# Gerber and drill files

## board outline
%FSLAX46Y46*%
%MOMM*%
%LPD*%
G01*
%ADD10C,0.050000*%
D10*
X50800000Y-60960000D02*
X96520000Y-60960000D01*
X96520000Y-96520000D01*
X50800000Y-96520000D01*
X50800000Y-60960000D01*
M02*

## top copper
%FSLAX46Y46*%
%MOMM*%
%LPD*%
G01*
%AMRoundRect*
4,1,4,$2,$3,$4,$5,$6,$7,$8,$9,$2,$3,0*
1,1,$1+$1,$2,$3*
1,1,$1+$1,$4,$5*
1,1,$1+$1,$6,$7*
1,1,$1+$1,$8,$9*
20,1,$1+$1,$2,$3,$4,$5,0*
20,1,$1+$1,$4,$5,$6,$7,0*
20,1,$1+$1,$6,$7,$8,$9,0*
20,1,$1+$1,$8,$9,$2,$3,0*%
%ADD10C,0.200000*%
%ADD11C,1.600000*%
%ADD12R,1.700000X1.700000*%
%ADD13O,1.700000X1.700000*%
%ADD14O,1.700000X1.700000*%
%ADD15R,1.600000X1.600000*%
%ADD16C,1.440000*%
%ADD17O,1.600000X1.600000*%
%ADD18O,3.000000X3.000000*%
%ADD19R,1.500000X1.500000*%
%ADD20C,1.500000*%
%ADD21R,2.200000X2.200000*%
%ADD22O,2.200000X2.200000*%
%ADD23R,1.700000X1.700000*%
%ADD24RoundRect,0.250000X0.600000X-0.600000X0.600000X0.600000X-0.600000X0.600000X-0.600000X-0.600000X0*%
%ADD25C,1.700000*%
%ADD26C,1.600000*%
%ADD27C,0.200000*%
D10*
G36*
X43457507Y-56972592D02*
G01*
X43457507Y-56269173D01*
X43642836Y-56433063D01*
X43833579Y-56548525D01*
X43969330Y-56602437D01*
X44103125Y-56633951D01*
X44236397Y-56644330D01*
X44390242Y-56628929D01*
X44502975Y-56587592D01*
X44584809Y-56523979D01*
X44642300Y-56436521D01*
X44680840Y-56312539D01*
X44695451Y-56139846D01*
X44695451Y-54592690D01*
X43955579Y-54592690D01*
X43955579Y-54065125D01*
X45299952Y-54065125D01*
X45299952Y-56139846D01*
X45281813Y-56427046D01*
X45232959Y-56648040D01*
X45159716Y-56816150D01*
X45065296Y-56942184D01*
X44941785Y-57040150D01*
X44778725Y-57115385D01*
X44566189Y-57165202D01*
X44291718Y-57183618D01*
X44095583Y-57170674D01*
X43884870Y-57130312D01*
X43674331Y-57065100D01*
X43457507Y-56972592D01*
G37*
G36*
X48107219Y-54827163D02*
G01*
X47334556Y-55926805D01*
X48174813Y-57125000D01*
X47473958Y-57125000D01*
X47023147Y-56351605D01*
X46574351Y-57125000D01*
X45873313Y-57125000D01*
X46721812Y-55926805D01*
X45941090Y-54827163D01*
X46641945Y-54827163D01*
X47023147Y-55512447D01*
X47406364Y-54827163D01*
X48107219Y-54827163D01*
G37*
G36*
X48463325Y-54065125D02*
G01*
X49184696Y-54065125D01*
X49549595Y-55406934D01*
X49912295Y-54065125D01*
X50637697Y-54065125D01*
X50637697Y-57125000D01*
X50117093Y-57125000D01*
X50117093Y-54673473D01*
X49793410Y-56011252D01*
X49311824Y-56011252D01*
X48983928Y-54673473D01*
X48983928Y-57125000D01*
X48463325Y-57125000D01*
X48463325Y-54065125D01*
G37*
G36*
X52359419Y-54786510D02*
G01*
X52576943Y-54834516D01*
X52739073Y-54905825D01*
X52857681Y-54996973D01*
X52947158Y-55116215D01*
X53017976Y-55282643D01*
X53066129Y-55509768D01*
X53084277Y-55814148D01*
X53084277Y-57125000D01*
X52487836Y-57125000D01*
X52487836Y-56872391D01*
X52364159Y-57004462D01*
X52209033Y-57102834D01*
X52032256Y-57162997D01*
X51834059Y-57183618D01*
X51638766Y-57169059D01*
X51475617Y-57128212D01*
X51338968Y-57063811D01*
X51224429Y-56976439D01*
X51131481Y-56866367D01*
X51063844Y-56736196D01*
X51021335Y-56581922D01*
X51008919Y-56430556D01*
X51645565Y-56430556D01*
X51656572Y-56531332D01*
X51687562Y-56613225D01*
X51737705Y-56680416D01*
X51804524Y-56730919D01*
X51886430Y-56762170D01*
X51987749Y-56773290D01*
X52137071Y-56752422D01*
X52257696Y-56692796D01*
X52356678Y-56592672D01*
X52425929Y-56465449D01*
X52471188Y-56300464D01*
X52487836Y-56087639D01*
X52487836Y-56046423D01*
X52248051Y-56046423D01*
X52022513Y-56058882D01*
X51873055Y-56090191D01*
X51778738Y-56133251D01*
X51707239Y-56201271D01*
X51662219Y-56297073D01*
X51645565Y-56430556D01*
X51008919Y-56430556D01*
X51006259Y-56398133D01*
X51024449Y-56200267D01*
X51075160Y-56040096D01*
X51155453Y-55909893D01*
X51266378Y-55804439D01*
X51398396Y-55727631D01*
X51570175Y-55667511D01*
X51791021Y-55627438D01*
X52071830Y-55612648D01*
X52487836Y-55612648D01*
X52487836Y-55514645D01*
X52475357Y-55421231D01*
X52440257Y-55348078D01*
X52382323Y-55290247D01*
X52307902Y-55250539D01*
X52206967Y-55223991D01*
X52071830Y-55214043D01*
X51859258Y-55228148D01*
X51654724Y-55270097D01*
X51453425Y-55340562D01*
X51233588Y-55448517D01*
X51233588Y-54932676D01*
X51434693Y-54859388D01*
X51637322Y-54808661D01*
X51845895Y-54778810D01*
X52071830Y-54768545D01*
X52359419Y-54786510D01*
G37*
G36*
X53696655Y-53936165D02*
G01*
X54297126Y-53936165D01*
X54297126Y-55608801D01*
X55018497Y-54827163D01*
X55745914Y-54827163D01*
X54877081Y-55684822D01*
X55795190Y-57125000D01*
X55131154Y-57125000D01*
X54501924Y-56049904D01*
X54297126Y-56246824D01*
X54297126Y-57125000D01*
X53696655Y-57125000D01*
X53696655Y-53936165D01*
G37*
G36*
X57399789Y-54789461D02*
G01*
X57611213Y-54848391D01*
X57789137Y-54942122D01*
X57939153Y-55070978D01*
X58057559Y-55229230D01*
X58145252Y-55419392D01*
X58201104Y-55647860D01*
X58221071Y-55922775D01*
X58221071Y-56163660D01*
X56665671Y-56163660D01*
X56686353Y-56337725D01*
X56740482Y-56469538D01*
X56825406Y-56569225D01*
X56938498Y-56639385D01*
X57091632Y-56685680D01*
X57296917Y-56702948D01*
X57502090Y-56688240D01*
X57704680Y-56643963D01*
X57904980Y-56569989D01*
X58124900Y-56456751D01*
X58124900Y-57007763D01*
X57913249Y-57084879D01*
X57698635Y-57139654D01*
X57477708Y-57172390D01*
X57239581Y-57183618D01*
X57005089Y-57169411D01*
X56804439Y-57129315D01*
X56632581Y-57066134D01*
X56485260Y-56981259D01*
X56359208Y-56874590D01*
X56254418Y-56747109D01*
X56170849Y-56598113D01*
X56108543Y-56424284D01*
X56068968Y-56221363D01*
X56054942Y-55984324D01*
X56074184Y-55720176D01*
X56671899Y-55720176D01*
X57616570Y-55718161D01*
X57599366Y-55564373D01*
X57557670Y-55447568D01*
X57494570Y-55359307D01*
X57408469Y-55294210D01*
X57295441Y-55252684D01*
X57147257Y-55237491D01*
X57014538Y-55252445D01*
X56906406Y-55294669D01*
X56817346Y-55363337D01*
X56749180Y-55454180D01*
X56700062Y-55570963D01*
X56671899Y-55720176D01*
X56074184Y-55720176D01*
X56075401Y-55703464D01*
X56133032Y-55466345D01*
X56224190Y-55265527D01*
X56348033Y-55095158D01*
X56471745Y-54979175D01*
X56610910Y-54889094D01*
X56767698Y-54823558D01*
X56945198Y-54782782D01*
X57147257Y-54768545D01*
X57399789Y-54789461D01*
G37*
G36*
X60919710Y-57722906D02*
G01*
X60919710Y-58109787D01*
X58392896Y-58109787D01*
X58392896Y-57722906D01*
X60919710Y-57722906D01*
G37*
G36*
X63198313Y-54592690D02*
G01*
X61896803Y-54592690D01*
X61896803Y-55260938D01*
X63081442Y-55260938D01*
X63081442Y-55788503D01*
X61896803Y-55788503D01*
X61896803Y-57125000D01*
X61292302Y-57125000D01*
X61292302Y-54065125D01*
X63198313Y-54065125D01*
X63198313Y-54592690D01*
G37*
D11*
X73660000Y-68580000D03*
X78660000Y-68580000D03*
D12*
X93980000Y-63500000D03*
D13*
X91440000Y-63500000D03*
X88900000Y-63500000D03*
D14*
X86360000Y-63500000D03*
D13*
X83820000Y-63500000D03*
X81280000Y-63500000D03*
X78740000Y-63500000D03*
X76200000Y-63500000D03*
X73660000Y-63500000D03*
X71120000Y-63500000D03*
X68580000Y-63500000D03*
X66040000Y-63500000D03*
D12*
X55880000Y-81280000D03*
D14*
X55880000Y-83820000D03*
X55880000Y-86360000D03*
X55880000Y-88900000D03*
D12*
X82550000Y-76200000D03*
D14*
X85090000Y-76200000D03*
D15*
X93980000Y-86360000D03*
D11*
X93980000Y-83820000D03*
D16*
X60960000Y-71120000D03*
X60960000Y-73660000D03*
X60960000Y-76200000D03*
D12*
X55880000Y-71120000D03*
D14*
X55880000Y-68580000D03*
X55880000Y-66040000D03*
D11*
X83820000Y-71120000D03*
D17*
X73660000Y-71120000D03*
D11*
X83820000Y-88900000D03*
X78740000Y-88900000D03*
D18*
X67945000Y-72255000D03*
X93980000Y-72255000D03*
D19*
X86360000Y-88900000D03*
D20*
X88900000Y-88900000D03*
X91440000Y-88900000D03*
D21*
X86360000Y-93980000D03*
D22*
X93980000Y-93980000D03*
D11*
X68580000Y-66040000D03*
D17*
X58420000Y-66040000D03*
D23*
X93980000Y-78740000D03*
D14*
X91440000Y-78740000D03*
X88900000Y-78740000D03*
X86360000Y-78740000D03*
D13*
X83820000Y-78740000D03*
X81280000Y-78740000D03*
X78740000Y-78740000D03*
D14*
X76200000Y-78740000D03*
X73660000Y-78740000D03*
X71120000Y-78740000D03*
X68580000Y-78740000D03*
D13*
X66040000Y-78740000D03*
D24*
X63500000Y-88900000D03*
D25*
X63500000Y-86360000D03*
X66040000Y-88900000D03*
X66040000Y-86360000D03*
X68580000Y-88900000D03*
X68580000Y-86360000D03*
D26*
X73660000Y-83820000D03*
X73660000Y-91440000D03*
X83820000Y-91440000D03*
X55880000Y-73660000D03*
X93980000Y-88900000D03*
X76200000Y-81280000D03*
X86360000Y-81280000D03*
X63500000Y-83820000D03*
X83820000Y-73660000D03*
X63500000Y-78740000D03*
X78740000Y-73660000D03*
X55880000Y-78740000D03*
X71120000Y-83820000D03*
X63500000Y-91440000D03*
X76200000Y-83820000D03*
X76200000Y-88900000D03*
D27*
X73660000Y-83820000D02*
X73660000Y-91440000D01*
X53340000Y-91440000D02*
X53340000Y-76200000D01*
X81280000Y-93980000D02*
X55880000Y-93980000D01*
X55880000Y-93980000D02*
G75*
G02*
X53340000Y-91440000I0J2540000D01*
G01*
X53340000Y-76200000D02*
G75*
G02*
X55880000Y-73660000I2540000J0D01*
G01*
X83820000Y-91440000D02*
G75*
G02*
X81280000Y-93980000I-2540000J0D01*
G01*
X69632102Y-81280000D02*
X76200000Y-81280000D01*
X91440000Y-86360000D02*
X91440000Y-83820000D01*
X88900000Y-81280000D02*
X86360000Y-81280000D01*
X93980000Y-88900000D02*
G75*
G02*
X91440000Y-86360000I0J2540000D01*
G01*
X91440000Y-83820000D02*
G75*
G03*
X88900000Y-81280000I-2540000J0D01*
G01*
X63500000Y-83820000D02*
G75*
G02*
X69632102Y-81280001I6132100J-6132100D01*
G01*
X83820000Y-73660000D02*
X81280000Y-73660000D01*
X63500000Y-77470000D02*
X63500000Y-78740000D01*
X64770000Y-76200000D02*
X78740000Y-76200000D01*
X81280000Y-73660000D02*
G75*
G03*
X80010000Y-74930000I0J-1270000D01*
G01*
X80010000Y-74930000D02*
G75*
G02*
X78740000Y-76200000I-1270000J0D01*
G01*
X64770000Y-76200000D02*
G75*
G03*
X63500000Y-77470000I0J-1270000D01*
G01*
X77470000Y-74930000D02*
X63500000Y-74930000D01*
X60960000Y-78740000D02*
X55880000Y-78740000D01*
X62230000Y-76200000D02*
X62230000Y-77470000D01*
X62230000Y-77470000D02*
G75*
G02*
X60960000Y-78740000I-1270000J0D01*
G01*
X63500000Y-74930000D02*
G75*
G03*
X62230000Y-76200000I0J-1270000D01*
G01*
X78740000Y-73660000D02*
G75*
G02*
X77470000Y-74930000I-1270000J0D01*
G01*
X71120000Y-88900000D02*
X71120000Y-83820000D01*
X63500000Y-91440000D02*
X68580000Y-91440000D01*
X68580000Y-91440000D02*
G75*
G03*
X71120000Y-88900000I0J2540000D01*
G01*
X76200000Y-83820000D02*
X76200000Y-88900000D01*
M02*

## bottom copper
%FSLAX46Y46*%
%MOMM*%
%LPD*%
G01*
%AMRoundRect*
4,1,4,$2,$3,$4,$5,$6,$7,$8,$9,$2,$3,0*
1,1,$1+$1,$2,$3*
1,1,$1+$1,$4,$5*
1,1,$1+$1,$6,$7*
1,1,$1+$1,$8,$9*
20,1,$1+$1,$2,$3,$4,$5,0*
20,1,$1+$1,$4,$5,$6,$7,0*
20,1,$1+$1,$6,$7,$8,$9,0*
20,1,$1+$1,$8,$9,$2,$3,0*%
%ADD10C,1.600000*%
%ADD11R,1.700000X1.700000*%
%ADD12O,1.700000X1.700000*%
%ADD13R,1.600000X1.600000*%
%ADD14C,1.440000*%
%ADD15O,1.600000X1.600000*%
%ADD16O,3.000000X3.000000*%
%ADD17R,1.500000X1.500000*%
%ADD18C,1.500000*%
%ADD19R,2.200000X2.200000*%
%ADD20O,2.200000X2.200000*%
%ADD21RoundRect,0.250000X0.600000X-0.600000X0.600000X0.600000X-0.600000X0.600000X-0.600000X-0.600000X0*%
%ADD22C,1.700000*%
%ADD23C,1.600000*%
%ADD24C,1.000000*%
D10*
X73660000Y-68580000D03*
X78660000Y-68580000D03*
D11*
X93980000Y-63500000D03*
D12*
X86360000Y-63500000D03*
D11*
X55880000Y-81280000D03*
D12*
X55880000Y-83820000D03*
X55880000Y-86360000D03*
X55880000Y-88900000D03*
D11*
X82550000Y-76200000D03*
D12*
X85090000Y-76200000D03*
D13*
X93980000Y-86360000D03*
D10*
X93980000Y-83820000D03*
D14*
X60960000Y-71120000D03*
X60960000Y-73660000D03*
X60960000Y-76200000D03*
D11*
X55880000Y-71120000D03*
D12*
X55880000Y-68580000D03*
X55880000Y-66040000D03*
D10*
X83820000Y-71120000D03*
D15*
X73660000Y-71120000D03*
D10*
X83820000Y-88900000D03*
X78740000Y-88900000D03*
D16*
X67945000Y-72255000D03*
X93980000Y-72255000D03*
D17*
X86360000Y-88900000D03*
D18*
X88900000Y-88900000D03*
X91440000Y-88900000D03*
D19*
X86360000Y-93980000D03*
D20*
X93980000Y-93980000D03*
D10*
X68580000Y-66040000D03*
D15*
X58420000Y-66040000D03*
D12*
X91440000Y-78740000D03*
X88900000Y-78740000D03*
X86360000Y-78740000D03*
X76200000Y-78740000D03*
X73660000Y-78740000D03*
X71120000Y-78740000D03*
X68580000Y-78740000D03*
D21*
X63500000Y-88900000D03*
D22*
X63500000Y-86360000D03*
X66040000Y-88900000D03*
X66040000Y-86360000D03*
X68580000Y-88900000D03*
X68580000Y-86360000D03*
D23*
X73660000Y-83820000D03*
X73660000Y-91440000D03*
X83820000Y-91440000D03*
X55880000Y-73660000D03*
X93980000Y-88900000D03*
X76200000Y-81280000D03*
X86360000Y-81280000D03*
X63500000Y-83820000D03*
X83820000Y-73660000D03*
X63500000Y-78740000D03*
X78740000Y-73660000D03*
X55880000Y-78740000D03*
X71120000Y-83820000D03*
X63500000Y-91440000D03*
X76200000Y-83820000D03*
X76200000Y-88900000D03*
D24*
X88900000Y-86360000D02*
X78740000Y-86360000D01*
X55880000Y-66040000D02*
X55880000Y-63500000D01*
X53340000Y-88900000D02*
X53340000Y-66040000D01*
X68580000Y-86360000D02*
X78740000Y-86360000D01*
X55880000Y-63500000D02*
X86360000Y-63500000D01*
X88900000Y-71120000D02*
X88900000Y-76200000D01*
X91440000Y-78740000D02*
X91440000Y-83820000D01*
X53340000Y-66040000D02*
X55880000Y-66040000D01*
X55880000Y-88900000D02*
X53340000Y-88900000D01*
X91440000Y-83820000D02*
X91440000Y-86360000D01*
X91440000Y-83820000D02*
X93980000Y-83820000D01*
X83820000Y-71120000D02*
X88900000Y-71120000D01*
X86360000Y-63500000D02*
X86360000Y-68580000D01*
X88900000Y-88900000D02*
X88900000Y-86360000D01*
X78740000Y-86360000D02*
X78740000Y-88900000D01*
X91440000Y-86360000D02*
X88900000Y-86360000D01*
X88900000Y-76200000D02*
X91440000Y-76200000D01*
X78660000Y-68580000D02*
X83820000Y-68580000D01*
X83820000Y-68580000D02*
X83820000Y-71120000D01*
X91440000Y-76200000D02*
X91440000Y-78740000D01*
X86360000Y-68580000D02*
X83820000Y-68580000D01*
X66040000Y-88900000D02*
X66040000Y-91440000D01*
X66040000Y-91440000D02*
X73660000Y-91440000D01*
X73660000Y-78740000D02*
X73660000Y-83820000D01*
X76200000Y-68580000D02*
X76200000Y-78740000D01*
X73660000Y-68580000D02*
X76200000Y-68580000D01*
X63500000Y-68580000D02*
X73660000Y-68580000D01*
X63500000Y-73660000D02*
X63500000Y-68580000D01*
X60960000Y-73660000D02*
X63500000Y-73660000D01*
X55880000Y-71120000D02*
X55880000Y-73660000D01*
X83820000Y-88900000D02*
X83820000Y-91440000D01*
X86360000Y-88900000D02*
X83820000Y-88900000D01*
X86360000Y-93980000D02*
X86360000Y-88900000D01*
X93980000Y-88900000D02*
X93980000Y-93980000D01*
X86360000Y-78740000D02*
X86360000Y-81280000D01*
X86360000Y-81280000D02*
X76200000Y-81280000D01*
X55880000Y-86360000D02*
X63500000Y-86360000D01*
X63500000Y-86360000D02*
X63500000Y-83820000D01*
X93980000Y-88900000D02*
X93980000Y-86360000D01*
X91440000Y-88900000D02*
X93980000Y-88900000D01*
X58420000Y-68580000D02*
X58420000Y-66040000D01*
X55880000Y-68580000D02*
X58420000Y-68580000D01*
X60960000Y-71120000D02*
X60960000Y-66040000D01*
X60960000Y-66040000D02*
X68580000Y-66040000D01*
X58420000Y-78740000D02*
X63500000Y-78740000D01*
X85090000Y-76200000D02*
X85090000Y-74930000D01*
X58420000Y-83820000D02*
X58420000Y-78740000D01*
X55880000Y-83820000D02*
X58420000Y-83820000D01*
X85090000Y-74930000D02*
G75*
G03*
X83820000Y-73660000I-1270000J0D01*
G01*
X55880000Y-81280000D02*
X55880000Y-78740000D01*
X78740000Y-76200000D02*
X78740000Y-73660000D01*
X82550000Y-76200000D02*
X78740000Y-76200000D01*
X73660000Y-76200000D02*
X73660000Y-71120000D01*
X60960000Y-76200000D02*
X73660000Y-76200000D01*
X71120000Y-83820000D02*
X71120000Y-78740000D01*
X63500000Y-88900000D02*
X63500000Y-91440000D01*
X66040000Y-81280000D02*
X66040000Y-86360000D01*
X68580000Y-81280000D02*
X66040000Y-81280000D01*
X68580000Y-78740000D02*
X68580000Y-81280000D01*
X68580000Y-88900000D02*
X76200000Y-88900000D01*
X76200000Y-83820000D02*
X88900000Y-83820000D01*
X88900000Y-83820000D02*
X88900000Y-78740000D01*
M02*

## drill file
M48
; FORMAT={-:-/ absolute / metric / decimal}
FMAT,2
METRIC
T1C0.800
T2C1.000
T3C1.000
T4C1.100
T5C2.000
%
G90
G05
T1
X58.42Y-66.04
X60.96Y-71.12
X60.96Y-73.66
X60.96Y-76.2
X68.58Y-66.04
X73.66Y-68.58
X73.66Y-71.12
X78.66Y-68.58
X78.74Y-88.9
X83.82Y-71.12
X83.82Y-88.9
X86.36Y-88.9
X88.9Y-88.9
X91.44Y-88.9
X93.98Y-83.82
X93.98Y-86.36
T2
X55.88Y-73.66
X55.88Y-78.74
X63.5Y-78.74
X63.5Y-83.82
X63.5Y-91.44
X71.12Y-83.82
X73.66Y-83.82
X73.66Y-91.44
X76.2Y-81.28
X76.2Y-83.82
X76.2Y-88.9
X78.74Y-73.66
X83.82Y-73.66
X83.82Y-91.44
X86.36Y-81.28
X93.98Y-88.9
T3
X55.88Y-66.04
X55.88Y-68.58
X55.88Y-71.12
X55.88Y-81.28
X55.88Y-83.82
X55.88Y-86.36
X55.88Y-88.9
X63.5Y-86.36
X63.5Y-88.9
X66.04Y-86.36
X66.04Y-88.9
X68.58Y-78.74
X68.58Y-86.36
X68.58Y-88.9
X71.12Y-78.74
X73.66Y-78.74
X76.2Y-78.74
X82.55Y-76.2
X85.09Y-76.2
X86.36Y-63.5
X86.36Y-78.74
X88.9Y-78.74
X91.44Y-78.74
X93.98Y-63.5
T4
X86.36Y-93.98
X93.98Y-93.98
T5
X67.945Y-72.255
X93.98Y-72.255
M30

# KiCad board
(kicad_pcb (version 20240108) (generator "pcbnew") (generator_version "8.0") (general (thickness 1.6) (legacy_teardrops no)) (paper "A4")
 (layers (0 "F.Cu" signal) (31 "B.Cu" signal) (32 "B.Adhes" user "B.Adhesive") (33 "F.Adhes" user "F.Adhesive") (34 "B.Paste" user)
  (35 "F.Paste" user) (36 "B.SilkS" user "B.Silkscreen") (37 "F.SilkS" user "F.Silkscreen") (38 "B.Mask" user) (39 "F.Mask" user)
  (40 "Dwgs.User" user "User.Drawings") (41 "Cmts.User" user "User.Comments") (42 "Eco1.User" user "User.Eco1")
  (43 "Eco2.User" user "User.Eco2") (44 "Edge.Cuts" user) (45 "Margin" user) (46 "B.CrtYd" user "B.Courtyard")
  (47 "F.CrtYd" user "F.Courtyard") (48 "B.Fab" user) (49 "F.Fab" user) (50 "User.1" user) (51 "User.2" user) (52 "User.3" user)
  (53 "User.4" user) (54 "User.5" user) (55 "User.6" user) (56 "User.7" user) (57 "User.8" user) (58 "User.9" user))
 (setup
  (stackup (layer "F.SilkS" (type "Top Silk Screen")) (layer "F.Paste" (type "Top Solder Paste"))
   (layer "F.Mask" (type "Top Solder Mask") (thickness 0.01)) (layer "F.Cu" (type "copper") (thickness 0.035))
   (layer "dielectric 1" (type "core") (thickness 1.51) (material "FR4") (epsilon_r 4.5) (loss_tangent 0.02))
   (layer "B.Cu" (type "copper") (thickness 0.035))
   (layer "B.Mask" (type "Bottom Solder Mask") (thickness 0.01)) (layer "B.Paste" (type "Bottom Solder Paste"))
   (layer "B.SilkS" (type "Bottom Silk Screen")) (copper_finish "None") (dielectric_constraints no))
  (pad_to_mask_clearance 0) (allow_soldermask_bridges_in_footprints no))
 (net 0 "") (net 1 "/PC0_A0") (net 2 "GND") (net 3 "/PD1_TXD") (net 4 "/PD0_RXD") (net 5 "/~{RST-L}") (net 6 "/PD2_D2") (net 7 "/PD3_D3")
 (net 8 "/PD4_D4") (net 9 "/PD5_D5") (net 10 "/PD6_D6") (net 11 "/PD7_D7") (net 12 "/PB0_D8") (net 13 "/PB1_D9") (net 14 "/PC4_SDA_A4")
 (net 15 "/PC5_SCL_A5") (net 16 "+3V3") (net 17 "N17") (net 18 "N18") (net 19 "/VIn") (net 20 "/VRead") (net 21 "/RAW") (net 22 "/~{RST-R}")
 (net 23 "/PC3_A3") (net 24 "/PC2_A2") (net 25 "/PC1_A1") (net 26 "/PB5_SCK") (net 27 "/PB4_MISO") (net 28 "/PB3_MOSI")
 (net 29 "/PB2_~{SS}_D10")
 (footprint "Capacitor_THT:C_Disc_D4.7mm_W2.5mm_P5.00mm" (layer "F.Cu") (at 73.66 68.58)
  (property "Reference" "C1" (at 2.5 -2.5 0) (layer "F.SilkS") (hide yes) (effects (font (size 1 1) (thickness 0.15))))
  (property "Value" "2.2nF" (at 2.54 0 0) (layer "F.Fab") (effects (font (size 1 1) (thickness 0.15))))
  (pad "1" thru_hole circle (at 0 0) (size 1.6 1.6) (drill 0.8) (layers "*.Cu" "*.Mask") (remove_unused_layers yes) (keep_end_layers yes)
   (zone_layer_connections) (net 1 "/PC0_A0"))
  (pad "2" thru_hole circle (at 5 0) (size 1.6 1.6) (drill 0.8) (layers "*.Cu" "*.Mask") (remove_unused_layers yes) (keep_end_layers yes)
   (zone_layer_connections) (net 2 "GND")))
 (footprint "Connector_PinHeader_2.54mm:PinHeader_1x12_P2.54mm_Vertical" (layer "F.Cu") (at 93.98 63.5 -90)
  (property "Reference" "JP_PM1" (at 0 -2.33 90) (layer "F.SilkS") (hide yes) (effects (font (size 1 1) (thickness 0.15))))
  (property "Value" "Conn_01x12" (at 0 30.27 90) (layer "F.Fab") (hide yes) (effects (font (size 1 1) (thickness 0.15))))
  (pad "1" thru_hole rect (at 0 0 270) (size 1.7 1.7) (drill 1) (layers "*.Cu" "*.Mask") (remove_unused_layers yes) (keep_end_layers yes)
   (zone_layer_connections) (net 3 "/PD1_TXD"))
  (pad "2" smd oval (at 0 2.54 270) (size 1.7 1.7) (layers "F.Cu" "F.Paste" "F.Mask") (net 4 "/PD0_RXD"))
  (pad "3" smd oval (at 0 5.08 270) (size 1.7 1.7) (layers "F.Cu" "F.Paste" "F.Mask") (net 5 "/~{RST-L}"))
  (pad "4" thru_hole oval (at 0 7.62 270) (size 1.7 1.7) (drill 1) (layers "*.Cu" "*.Mask") (remove_unused_layers yes) (keep_end_layers yes)
   (zone_layer_connections) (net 2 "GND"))
  (pad "5" smd oval (at 0 10.16 270) (size 1.7 1.7) (layers "F.Cu" "F.Paste" "F.Mask") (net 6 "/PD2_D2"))
  (pad "6" smd oval (at 0 12.7 270) (size 1.7 1.7) (layers "F.Cu" "F.Paste" "F.Mask") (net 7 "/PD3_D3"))
  (pad "7" smd oval (at 0 15.24 270) (size 1.7 1.7) (layers "F.Cu" "F.Paste" "F.Mask") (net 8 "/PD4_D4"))
  (pad "8" smd oval (at 0 17.78 270) (size 1.7 1.7) (layers "F.Cu" "F.Paste" "F.Mask") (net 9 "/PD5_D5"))
  (pad "9" smd oval (at 0 20.32 270) (size 1.7 1.7) (layers "F.Cu" "F.Paste" "F.Mask") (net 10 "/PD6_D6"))
  (pad "10" smd oval (at 0 22.86 270) (size 1.7 1.7) (layers "F.Cu" "F.Paste" "F.Mask") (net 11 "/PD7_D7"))
  (pad "11" smd oval (at 0 25.4 270) (size 1.7 1.7) (layers "F.Cu" "F.Paste" "F.Mask") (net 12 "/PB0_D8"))
  (pad "12" smd oval (at 0 27.94 270) (size 1.7 1.7) (layers "F.Cu" "F.Paste" "F.Mask") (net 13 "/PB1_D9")))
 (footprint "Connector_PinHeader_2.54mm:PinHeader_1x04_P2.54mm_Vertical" (layer "F.Cu") (at 55.88 81.28)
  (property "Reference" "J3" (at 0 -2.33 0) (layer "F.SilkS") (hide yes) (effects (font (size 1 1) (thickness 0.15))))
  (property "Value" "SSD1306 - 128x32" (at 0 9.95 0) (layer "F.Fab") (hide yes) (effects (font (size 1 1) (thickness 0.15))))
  (pad "1" thru_hole rect (at 0 0) (size 1.7 1.7) (drill 1) (layers "*.Cu" "*.Mask") (remove_unused_layers yes) (keep_end_layers yes)
   (zone_layer_connections) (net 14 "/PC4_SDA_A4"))
  (pad "2" thru_hole oval (at 0 2.54) (size 1.7 1.7) (drill 1) (layers "*.Cu" "*.Mask") (remove_unused_layers yes) (keep_end_layers yes)
   (zone_layer_connections) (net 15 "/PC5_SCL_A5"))
  (pad "3" thru_hole oval (at 0 5.08) (size 1.7 1.7) (drill 1) (layers "*.Cu" "*.Mask") (remove_unused_layers yes) (keep_end_layers yes)
   (zone_layer_connections) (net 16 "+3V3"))
  (pad "4" thru_hole oval (at 0 7.62) (size 1.7 1.7) (drill 1) (layers "*.Cu" "*.Mask") (remove_unused_layers yes) (keep_end_layers yes)
   (zone_layer_connections) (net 2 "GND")))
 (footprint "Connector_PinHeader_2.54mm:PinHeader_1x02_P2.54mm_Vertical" (layer "F.Cu") (at 82.55 76.2 90)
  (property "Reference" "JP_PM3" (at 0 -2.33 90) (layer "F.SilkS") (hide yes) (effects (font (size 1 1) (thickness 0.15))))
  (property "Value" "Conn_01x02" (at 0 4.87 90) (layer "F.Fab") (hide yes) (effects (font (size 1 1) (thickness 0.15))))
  (pad "1" thru_hole rect (at 0 0 90) (size 1.7 1.7) (drill 1) (layers "*.Cu" "*.Mask") (remove_unused_layers yes) (keep_end_layers yes)
   (zone_layer_connections) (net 14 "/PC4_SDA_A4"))
  (pad "2" thru_hole oval (at 0 2.54 90) (size 1.7 1.7) (drill 1) (layers "*.Cu" "*.Mask") (remove_unused_layers yes) (keep_end_layers yes)
   (zone_layer_connections) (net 15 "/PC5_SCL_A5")))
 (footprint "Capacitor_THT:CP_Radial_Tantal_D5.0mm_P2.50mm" (layer "F.Cu") (at 93.98 86.36 90)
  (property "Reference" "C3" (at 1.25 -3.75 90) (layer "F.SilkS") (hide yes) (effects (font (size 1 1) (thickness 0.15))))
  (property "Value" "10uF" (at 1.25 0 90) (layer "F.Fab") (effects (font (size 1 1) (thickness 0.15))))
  (pad "1" thru_hole rect (at 0 0 90) (size 1.6 1.6) (drill 0.8) (layers "*.Cu" "*.Mask") (remove_unused_layers yes) (keep_end_layers yes)
   (zone_layer_connections) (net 16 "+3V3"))
  (pad "2" thru_hole circle (at 2.54 0 90) (size 1.6 1.6) (drill 0.8) (layers "*.Cu" "*.Mask") (remove_unused_layers yes)
   (keep_end_layers yes) (zone_layer_connections) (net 2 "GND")))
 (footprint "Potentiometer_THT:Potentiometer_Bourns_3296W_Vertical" (layer "F.Cu") (at 60.96 71.12 90)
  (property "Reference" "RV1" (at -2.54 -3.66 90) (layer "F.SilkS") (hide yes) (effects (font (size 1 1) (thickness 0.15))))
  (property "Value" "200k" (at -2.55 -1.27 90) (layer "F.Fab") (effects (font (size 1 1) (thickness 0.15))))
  (pad "1" thru_hole circle (at 0 0 90) (size 1.44 1.44) (drill 0.8) (layers "*.Cu" "*.Mask") (remove_unused_layers yes)
   (keep_end_layers yes) (zone_layer_connections) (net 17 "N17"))
  (pad "2" thru_hole circle (at -2.54 0 90) (size 1.44 1.44) (drill 0.8) (layers "*.Cu" "*.Mask") (remove_unused_layers yes)
   (keep_end_layers yes) (zone_layer_connections) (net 1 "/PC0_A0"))
  (pad "3" thru_hole circle (at -5.08 0 90) (size 1.44 1.44) (drill 0.8) (layers "*.Cu" "*.Mask") (remove_unused_layers yes)
   (keep_end_layers yes) (zone_layer_connections) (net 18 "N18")))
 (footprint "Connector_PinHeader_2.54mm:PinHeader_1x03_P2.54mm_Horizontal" (layer "F.Cu") (at 55.88 71.12 180)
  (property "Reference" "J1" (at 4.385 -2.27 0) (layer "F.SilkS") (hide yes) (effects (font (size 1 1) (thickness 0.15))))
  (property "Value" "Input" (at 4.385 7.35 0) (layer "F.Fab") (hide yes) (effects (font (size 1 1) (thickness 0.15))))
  (pad "1" thru_hole rect (at 0 0 180) (size 1.7 1.7) (drill 1) (layers "*.Cu" "*.Mask") (remove_unused_layers yes) (keep_end_layers yes)
   (zone_layer_connections) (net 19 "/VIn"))
  (pad "2" thru_hole oval (at 0 2.54 180) (size 1.7 1.7) (drill 1) (layers "*.Cu" "*.Mask") (remove_unused_layers yes) (keep_end_layers yes)
   (zone_layer_connections) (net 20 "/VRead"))
  (pad "3" thru_hole oval (at 0 5.08 180) (size 1.7 1.7) (drill 1) (layers "*.Cu" "*.Mask") (remove_unused_layers yes) (keep_end_layers yes)
   (zone_layer_connections) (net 2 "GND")))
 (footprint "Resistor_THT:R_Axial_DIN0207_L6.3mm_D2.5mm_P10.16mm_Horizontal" (layer "F.Cu") (at 83.82 71.12 180)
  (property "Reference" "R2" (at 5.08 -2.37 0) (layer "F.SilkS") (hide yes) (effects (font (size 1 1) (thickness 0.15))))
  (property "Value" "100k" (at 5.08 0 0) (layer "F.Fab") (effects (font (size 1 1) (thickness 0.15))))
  (pad "1" thru_hole circle (at 0 0 180) (size 1.6 1.6) (drill 0.8) (layers "*.Cu" "*.Mask") (remove_unused_layers yes)
   (keep_end_layers yes) (zone_layer_connections) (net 2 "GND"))
  (pad "2" thru_hole oval (at 10.16 0 180) (size 1.6 1.6) (drill 0.8) (layers "*.Cu" "*.Mask") (remove_unused_layers yes)
   (keep_end_layers yes) (zone_layer_connections) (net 18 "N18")))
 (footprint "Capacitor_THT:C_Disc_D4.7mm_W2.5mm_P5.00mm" (layer "F.Cu") (at 83.82 88.9 180)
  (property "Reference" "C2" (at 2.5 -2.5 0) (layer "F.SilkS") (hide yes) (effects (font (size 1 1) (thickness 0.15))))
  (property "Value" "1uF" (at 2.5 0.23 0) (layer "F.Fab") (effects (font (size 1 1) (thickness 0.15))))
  (pad "1" thru_hole circle (at 0 0 180) (size 1.6 1.6) (drill 0.8) (layers "*.Cu" "*.Mask") (remove_unused_layers yes)
   (keep_end_layers yes) (zone_layer_connections) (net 19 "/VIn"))
  (pad "2" thru_hole circle (at 5.08 0 180) (size 1.6 1.6) (drill 0.8) (layers "*.Cu" "*.Mask") (remove_unused_layers yes)
   (keep_end_layers yes) (zone_layer_connections) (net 2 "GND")))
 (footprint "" (layer "F.Cu") (at 67.945 72.255)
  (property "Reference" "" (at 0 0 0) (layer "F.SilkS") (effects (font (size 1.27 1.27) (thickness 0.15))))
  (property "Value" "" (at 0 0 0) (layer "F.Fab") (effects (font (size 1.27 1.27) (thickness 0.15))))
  (pad "1" thru_hole oval (at 0 0 90) (size 3 3) (drill 2) (layers "*.Cu" "*.Mask") (remove_unused_layers yes) (keep_end_layers yes)
   (zone_layer_connections))
  (pad "2" thru_hole oval (at 26.035 0 90) (size 3 3) (drill 2) (layers "*.Cu" "*.Mask") (remove_unused_layers yes) (keep_end_layers yes)
   (zone_layer_connections)))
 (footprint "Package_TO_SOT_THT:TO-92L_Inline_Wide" (layer "F.Cu") (at 86.36 88.9)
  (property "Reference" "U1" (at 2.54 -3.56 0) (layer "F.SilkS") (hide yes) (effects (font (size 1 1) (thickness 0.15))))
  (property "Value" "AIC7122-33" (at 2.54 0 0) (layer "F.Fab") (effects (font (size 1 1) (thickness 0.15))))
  (pad "1" thru_hole rect (at 0 0) (size 1.5 1.5) (drill 0.8) (layers "*.Cu" "*.Mask") (remove_unused_layers yes) (keep_end_layers yes)
   (zone_layer_connections) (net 19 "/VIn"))
  (pad "2" thru_hole circle (at 2.54 0) (size 1.5 1.5) (drill 0.8) (layers "*.Cu" "*.Mask") (remove_unused_layers yes) (keep_end_layers yes)
   (zone_layer_connections) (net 2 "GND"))
  (pad "3" thru_hole circle (at 5.08 0) (size 1.5 1.5) (drill 0.8) (layers "*.Cu" "*.Mask") (remove_unused_layers yes) (keep_end_layers yes)
   (zone_layer_connections) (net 16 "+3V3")))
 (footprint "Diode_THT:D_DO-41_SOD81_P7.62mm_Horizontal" (layer "F.Cu") (at 86.36 93.98)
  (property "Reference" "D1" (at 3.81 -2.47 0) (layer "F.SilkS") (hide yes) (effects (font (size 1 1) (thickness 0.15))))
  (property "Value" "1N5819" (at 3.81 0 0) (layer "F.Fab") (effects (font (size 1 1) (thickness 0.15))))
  (pad "1" thru_hole rect (at 0 0) (size 2.2 2.2) (drill 1.1) (layers "*.Cu" "*.Mask") (remove_unused_layers no) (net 19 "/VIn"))
  (pad "2" thru_hole oval (at 7.62 0) (size 2.2 2.2) (drill 1.1) (layers "*.Cu" "*.Mask") (remove_unused_layers no) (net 16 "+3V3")))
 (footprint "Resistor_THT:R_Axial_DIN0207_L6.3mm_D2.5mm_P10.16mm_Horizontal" (layer "F.Cu") (at 68.58 66.04 180)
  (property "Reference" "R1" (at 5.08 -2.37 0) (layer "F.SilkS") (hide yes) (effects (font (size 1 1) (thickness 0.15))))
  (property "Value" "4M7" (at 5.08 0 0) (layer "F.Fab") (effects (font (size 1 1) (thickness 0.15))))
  (pad "1" thru_hole circle (at 0 0 180) (size 1.6 1.6) (drill 0.8) (layers "*.Cu" "*.Mask") (remove_unused_layers yes)
   (keep_end_layers yes) (zone_layer_connections) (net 17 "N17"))
  (pad "2" thru_hole oval (at 10.16 0 180) (size 1.6 1.6) (drill 0.8) (layers "*.Cu" "*.Mask") (remove_unused_layers yes)
   (keep_end_layers yes) (zone_layer_connections) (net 20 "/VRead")))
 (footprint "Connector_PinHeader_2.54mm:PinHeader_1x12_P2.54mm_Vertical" (layer "F.Cu") (at 93.98 78.74 -90)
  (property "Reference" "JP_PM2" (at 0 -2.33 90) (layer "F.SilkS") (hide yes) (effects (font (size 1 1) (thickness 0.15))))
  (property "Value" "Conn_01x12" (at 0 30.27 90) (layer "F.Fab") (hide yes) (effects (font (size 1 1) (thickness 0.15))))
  (pad "1" smd rect (at 0 0 270) (size 1.7 1.7) (layers "F.Cu" "F.Paste" "F.Mask") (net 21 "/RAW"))
  (pad "2" thru_hole oval (at 0 2.54 270) (size 1.7 1.7) (drill 1) (layers "*.Cu" "*.Mask") (remove_unused_layers yes) (keep_end_layers yes)
   (zone_layer_connections) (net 2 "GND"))
  (pad "3" thru_hole oval (at 0 5.08 270) (size 1.7 1.7) (drill 1) (layers "*.Cu" "*.Mask") (remove_unused_layers yes) (keep_end_layers yes)
   (zone_layer_connections) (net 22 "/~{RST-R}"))
  (pad "4" thru_hole oval (at 0 7.62 270) (size 1.7 1.7) (drill 1) (layers "*.Cu" "*.Mask") (remove_unused_layers yes) (keep_end_layers yes)
   (zone_layer_connections) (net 16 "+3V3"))
  (pad "5" smd oval (at 0 10.16 270) (size 1.7 1.7) (layers "F.Cu" "F.Paste" "F.Mask") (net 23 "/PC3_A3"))
  (pad "6" smd oval (at 0 12.7 270) (size 1.7 1.7) (layers "F.Cu" "F.Paste" "F.Mask") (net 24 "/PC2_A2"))
  (pad "7" smd oval (at 0 15.24 270) (size 1.7 1.7) (layers "F.Cu" "F.Paste" "F.Mask") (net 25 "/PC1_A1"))
  (pad "8" thru_hole oval (at 0 17.78 270) (size 1.7 1.7) (drill 1) (layers "*.Cu" "*.Mask") (remove_unused_layers yes)
   (keep_end_layers yes) (zone_layer_connections) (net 1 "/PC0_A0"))
  (pad "9" thru_hole oval (at 0 20.32 270) (size 1.7 1.7) (drill 1) (layers "*.Cu" "*.Mask") (remove_unused_layers yes)
   (keep_end_layers yes) (zone_layer_connections) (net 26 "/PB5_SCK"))
  (pad "10" thru_hole oval (at 0 22.86 270) (size 1.7 1.7) (drill 1) (layers "*.Cu" "*.Mask") (remove_unused_layers yes)
   (keep_end_layers yes) (zone_layer_connections) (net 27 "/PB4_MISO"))
  (pad "11" thru_hole oval (at 0 25.4 270) (size 1.7 1.7) (drill 1) (layers "*.Cu" "*.Mask") (remove_unused_layers yes)
   (keep_end_layers yes) (zone_layer_connections) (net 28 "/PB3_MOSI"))
  (pad "12" smd oval (at 0 27.94 270) (size 1.7 1.7) (layers "F.Cu" "F.Paste" "F.Mask") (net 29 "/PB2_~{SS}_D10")))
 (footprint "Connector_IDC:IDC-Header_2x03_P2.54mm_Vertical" (layer "F.Cu") (at 63.5 88.9 90)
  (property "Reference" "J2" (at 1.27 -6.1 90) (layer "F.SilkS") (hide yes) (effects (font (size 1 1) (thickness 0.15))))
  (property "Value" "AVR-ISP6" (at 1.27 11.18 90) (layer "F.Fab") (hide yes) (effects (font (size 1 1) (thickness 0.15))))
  (pad "1" thru_hole roundrect (at 0 0 90) (size 1.7 1.7) (drill 1) (layers "*.Cu" "*.Mask") (remove_unused_layers yes)
   (keep_end_layers yes) (zone_layer_connections) (roundrect_rratio 0.147059) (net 27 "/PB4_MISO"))
  (pad "2" thru_hole circle (at 2.54 0 90) (size 1.7 1.7) (drill 1) (layers "*.Cu" "*.Mask") (remove_unused_layers yes)
   (keep_end_layers yes) (zone_layer_connections) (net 16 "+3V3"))
  (pad "3" thru_hole circle (at 0 2.54 90) (size 1.7 1.7) (drill 1) (layers "*.Cu" "*.Mask") (remove_unused_layers yes)
   (keep_end_layers yes) (zone_layer_connections) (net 26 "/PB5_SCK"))
  (pad "4" thru_hole circle (at 2.54 2.54 90) (size 1.7 1.7) (drill 1) (layers "*.Cu" "*.Mask") (remove_unused_layers yes)
   (keep_end_layers yes) (zone_layer_connections) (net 28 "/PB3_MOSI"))
  (pad "5" thru_hole circle (at 0 5.08 90) (size 1.7 1.7) (drill 1) (layers "*.Cu" "*.Mask") (remove_unused_layers yes)
   (keep_end_layers yes) (zone_layer_connections) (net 22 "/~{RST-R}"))
  (pad "6" thru_hole circle (at 2.54 5.08 90) (size 1.7 1.7) (drill 1) (layers "*.Cu" "*.Mask") (remove_unused_layers yes)
   (keep_end_layers yes) (zone_layer_connections) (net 2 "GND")))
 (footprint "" (layer "F.Cu") (at 106.553 77.851)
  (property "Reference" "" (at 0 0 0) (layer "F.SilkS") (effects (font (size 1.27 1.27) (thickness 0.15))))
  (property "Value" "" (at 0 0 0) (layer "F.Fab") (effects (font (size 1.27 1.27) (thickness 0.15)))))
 (gr_rect (start 50.8 60.96) (end 96.52 96.52) (stroke (width 0.05) (type default)) (fill none) (layer "Edge.Cuts"))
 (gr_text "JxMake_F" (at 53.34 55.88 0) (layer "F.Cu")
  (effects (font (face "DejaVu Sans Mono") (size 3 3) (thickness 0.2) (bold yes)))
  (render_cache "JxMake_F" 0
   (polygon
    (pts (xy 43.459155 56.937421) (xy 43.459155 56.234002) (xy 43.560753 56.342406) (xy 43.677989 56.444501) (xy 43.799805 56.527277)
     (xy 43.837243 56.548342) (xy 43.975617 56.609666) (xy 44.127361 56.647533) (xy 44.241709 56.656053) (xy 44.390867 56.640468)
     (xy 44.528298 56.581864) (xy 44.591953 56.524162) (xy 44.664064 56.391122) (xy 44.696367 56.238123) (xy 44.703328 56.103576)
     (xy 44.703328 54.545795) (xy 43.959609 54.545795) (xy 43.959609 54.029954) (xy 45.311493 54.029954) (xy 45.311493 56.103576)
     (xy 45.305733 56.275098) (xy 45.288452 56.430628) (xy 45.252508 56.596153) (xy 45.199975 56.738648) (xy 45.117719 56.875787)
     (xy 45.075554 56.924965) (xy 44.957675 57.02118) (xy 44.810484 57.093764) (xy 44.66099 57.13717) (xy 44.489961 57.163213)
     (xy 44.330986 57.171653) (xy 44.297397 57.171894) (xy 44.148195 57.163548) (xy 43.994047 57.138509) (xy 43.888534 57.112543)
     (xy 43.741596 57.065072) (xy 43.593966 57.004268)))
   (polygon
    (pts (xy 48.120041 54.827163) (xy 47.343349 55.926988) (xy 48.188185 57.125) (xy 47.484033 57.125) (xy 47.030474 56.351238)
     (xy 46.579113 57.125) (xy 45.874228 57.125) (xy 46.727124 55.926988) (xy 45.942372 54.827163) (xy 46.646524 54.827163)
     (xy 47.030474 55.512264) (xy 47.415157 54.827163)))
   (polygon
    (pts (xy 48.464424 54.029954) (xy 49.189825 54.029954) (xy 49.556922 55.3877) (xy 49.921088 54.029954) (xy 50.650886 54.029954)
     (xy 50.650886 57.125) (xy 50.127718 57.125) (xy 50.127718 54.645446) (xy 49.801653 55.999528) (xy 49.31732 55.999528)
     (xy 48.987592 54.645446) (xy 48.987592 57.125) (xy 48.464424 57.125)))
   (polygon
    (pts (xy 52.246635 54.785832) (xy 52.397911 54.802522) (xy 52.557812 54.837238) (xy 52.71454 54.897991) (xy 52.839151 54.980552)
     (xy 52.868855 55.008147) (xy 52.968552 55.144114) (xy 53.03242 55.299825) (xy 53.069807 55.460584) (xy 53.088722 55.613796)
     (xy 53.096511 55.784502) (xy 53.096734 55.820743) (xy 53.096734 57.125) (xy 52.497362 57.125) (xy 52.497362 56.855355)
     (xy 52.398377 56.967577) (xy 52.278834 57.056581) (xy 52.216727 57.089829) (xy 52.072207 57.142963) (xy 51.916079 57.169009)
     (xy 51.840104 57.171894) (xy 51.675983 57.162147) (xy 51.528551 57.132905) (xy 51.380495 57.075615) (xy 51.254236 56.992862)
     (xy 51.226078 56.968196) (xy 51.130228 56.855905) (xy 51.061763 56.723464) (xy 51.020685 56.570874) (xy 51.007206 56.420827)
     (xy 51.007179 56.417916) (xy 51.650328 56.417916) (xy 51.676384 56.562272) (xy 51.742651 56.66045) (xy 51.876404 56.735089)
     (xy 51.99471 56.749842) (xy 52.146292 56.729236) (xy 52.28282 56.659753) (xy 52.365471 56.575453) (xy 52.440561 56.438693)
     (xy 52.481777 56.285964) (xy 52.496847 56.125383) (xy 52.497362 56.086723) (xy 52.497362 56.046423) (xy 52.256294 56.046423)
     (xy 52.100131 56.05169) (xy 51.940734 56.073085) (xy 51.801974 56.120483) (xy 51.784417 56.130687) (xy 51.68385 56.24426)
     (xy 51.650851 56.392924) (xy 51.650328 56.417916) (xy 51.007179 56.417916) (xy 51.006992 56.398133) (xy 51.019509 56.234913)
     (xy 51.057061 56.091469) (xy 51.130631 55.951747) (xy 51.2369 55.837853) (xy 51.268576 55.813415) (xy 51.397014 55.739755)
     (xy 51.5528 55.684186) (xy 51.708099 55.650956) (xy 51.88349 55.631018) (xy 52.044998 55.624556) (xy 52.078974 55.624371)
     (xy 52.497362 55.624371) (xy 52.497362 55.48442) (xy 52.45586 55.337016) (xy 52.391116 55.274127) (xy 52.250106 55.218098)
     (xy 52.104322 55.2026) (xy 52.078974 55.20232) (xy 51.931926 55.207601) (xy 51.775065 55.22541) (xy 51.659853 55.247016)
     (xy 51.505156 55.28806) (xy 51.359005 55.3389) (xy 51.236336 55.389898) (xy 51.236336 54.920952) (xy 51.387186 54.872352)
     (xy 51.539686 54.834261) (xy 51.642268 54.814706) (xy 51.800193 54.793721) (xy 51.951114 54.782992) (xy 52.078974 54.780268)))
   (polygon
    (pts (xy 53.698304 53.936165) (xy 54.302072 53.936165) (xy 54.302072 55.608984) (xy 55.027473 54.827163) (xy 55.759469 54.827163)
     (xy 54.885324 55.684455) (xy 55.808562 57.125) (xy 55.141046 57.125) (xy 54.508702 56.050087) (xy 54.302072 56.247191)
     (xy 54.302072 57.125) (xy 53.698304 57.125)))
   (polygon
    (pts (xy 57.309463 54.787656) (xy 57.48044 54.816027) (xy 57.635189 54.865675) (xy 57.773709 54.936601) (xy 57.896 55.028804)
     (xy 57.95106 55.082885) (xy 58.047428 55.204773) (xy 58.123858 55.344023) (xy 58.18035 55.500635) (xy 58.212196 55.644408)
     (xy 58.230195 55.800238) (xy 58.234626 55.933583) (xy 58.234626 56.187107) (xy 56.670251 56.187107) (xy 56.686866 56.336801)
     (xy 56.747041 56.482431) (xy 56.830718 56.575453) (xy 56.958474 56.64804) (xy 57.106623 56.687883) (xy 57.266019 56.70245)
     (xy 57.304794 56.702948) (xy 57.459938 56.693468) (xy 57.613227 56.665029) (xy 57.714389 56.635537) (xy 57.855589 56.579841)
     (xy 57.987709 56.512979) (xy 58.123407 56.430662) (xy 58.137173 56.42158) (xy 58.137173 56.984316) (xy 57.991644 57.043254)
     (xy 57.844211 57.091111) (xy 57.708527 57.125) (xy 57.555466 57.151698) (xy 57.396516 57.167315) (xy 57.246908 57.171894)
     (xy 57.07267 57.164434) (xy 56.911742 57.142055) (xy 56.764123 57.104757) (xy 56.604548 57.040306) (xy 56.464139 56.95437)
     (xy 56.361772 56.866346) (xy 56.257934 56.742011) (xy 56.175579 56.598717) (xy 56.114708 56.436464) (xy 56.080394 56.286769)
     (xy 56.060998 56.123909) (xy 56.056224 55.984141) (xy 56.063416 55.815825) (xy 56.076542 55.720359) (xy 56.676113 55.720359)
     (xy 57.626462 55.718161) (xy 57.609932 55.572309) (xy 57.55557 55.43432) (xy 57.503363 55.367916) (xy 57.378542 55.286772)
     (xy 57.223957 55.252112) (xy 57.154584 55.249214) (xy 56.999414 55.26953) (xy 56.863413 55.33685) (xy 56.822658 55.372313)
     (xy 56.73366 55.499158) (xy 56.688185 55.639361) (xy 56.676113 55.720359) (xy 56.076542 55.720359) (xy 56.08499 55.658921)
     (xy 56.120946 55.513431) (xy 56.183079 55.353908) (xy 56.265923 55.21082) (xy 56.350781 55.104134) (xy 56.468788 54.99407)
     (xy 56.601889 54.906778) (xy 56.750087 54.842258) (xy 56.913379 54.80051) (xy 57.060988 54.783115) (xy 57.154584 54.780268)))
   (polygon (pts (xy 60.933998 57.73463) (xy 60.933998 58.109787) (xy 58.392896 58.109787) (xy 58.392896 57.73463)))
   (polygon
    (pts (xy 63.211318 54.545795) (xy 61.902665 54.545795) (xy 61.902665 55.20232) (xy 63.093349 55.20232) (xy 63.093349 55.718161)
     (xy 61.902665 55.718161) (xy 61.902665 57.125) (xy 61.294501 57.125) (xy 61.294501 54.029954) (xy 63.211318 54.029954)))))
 (segment (start 88.9 86.36) (end 78.74 86.36) (width 1) (layer "B.Cu") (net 2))
 (segment (start 55.88 66.04) (end 55.88 63.5) (width 1) (layer "B.Cu") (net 2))
 (segment (start 53.34 88.9) (end 53.34 66.04) (width 1) (layer "B.Cu") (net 2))
 (segment (start 68.58 86.36) (end 78.74 86.36) (width 1) (layer "B.Cu") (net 2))
 (segment (start 55.88 63.5) (end 86.36 63.5) (width 1) (layer "B.Cu") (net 2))
 (segment (start 88.9 71.12) (end 88.9 76.2) (width 1) (layer "B.Cu") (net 2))
 (segment (start 91.44 78.74) (end 91.44 83.82) (width 1) (layer "B.Cu") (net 2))
 (segment (start 53.34 66.04) (end 55.88 66.04) (width 1) (layer "B.Cu") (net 2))
 (segment (start 55.88 88.9) (end 53.34 88.9) (width 1) (layer "B.Cu") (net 2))
 (segment (start 91.44 83.82) (end 91.44 86.36) (width 1) (layer "B.Cu") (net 2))
 (segment (start 91.44 83.82) (end 93.98 83.82) (width 1) (layer "B.Cu") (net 2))
 (segment (start 83.82 71.12) (end 88.9 71.12) (width 1) (layer "B.Cu") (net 2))
 (segment (start 86.36 63.5) (end 86.36 68.58) (width 1) (layer "B.Cu") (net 2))
 (segment (start 88.9 88.9) (end 88.9 86.36) (width 1) (layer "B.Cu") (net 2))
 (segment (start 78.74 86.36) (end 78.74 88.9) (width 1) (layer "B.Cu") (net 2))
 (segment (start 91.44 86.36) (end 88.9 86.36) (width 1) (layer "B.Cu") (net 2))
 (segment (start 88.9 76.2) (end 91.44 76.2) (width 1) (layer "B.Cu") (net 2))
 (segment (start 78.66 68.58) (end 83.82 68.58) (width 1) (layer "B.Cu") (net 2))
 (segment (start 83.82 68.58) (end 83.82 71.12) (width 1) (layer "B.Cu") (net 2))
 (segment (start 91.44 76.2) (end 91.44 78.74) (width 1) (layer "B.Cu") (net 2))
 (segment (start 86.36 68.58) (end 83.82 68.58) (width 1) (layer "B.Cu") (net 2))
 (segment (start 73.66 83.82) (end 73.66 91.44) (width 0.2) (layer "F.Cu") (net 26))
 (via (at 73.66 83.82) (size 1.6) (drill 1) (layers "F.Cu" "B.Cu") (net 26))
 (via (at 73.66 91.44) (size 1.6) (drill 1) (layers "F.Cu" "B.Cu") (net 26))
 (segment (start 66.04 88.9) (end 66.04 91.44) (width 1) (layer "B.Cu") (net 26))
 (segment (start 66.04 91.44) (end 73.66 91.44) (width 1) (layer "B.Cu") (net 26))
 (segment (start 73.66 78.74) (end 73.66 83.82) (width 1) (layer "B.Cu") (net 26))
 (segment (start 76.2 68.58) (end 76.2 78.74) (width 1) (layer "B.Cu") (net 1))
 (segment (start 73.66 68.58) (end 76.2 68.58) (width 1) (layer "B.Cu") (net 1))
 (segment (start 63.5 68.58) (end 73.66 68.58) (width 1) (layer "B.Cu") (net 1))
 (segment (start 63.5 73.66) (end 63.5 68.58) (width 1) (layer "B.Cu") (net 1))
 (segment (start 60.96 73.66) (end 63.5 73.66) (width 1) (layer "B.Cu") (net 1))
 (segment (start 53.34 91.44) (end 53.34 76.2) (width 0.2) (layer "F.Cu") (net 19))
 (segment (start 81.28 93.98) (end 55.88 93.98) (width 0.2) (layer "F.Cu") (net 19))
 (via (at 83.82 91.44) (size 1.6) (drill 1) (layers "F.Cu" "B.Cu") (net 19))
 (via (at 55.88 73.66) (size 1.6) (drill 1) (layers "F.Cu" "B.Cu") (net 19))
 (arc (start 55.88 93.98) (mid 54.083949 93.236051) (end 53.34 91.44) (width 0.2) (layer "F.Cu") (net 19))
 (arc (start 53.34 76.2) (mid 54.083949 74.403949) (end 55.88 73.66) (width 0.2) (layer "F.Cu") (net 19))
 (arc (start 83.82 91.44) (mid 83.076051 93.236051) (end 81.28 93.98) (width 0.2) (layer "F.Cu") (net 19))
 (segment (start 55.88 71.12) (end 55.88 73.66) (width 1) (layer "B.Cu") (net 19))
 (segment (start 83.82 88.9) (end 83.82 91.44) (width 1) (layer "B.Cu") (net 19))
 (segment (start 86.36 88.9) (end 83.82 88.9) (width 1) (layer "B.Cu") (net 19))
 (segment (start 86.36 93.98) (end 86.36 88.9) (width 1) (layer "B.Cu") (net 19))
 (segment (start 69.632102 81.28) (end 76.2 81.28) (width 0.2) (layer "F.Cu") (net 16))
 (segment (start 91.44 86.36) (end 91.44 83.82) (width 0.2) (layer "F.Cu") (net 16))
 (segment (start 88.9 81.28) (end 86.36 81.28) (width 0.2) (layer "F.Cu") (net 16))
 (via (at 93.98 88.9) (size 1.6) (drill 1) (layers "F.Cu" "B.Cu") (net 16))
 (via (at 76.2 81.28) (size 1.6) (drill 1) (layers "F.Cu" "B.Cu") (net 16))
 (via (at 86.36 81.28) (size 1.6) (drill 1) (layers "F.Cu" "B.Cu") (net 16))
 (via (at 63.5 83.82) (size 1.6) (drill 1) (layers "F.Cu" "B.Cu") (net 16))
 (arc (start 93.98 88.9) (mid 92.183949 88.156051) (end 91.44 86.36) (width 0.2) (layer "F.Cu") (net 16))
 (arc (start 91.44 83.82) (mid 90.696051 82.023949) (end 88.9 81.28) (width 0.2) (layer "F.Cu") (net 16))
 (arc (start 63.5 83.82) (mid 66.313432 81.940125) (end 69.632102 81.28) (width 0.2) (layer "F.Cu") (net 16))
 (segment (start 93.98 88.9) (end 93.98 93.98) (width 1) (layer "B.Cu") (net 16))
 (segment (start 86.36 78.74) (end 86.36 81.28) (width 1) (layer "B.Cu") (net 16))
 (segment (start 86.36 81.28) (end 76.2 81.28) (width 1) (layer "B.Cu") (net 16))
 (segment (start 55.88 86.36) (end 63.5 86.36) (width 1) (layer "B.Cu") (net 16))
 (segment (start 63.5 86.36) (end 63.5 83.82) (width 1) (layer "B.Cu") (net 16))
 (segment (start 93.98 88.9) (end 93.98 86.36) (width 1) (layer "B.Cu") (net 16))
 (segment (start 91.44 88.9) (end 93.98 88.9) (width 1) (layer "B.Cu") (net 16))
 (segment (start 58.42 68.58) (end 58.42 66.04) (width 1) (layer "B.Cu") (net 20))
 (segment (start 55.88 68.58) (end 58.42 68.58) (width 1) (layer "B.Cu") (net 20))
 (segment (start 60.96 71.12) (end 60.96 66.04) (width 1) (layer "B.Cu") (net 17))
 (segment (start 60.96 66.04) (end 68.58 66.04) (width 1) (layer "B.Cu") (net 17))
 (segment (start 83.82 73.66) (end 81.28 73.66) (width 0.2) (layer "F.Cu") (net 15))
 (segment (start 63.5 77.47) (end 63.5 78.74) (width 0.2) (layer "F.Cu") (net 15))
 (segment (start 64.77 76.2) (end 78.74 76.2) (width 0.2) (layer "F.Cu") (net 15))
 (via (at 83.82 73.66) (size 1.6) (drill 1) (layers "F.Cu" "B.Cu") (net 15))
 (via (at 63.5 78.74) (size 1.6) (drill 1) (layers "F.Cu" "B.Cu") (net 15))
 (arc (start 81.28 73.66) (mid 80.381974 74.031974) (end 80.01 74.93) (width 0.2) (layer "F.Cu") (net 15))
 (arc (start 80.01 74.93) (mid 79.638026 75.828026) (end 78.74 76.2) (width 0.2) (layer "F.Cu") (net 15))
 (arc (start 64.77 76.2) (mid 63.871974 76.571974) (end 63.5 77.47) (width 0.2) (layer "F.Cu") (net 15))
 (segment (start 58.42 78.74) (end 63.5 78.74) (width 1) (layer "B.Cu") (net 15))
 (segment (start 85.09 76.2) (end 85.09 74.93) (width 1) (layer "B.Cu") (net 15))
 (segment (start 58.42 83.82) (end 58.42 78.74) (width 1) (layer "B.Cu") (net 15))
 (segment (start 55.88 83.82) (end 58.42 83.82) (width 1) (layer "B.Cu") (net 15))
 (arc (start 85.09 74.93) (mid 84.718026 74.031974) (end 83.82 73.66) (width 1) (layer "B.Cu") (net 15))
 (segment (start 77.47 74.93) (end 63.5 74.93) (width 0.2) (layer "F.Cu") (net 14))
 (segment (start 60.96 78.74) (end 55.88 78.74) (width 0.2) (layer "F.Cu") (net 14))
 (segment (start 62.23 76.2) (end 62.23 77.47) (width 0.2) (layer "F.Cu") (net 14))
 (via (at 78.74 73.66) (size 1.6) (drill 1) (layers "F.Cu" "B.Cu") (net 14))
 (via (at 55.88 78.74) (size 1.6) (drill 1) (layers "F.Cu" "B.Cu") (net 14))
 (arc (start 62.23 77.47) (mid 61.858026 78.368026) (end 60.96 78.74) (width 0.2) (layer "F.Cu") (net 14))
 (arc (start 63.5 74.93) (mid 62.601974 75.301974) (end 62.23 76.2) (width 0.2) (layer "F.Cu") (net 14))
 (arc (start 78.74 73.66) (mid 78.368026 74.558026) (end 77.47 74.93) (width 0.2) (layer "F.Cu") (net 14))
 (segment (start 55.88 81.28) (end 55.88 78.74) (width 1) (layer "B.Cu") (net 14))
 (segment (start 78.74 76.2) (end 78.74 73.66) (width 1) (layer "B.Cu") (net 14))
 (segment (start 82.55 76.2) (end 78.74 76.2) (width 1) (layer "B.Cu") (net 14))
 (segment (start 73.66 76.2) (end 73.66 71.12) (width 1) (layer "B.Cu") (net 18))
 (segment (start 60.96 76.2) (end 73.66 76.2) (width 1) (layer "B.Cu") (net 18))
 (segment (start 71.12 88.9) (end 71.12 83.82) (width 0.2) (layer "F.Cu") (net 27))
 (segment (start 63.5 91.44) (end 68.58 91.44) (width 0.2) (layer "F.Cu") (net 27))
 (via (at 71.12 83.82) (size 1.6) (drill 1) (layers "F.Cu" "B.Cu") (free yes) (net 27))
 (via (at 63.5 91.44) (size 1.6) (drill 1) (layers "F.Cu" "B.Cu") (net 27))
 (arc (start 68.58 91.44) (mid 70.376051 90.696051) (end 71.12 88.9) (width 0.2) (layer "F.Cu") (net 27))
 (segment (start 71.12 83.82) (end 71.12 78.74) (width 1) (layer "B.Cu") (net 27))
 (segment (start 63.5 88.9) (end 63.5 91.44) (width 1) (layer "B.Cu") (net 27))
 (segment (start 66.04 81.28) (end 66.04 86.36) (width 1) (layer "B.Cu") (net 28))
 (segment (start 68.58 81.28) (end 66.04 81.28) (width 1) (layer "B.Cu") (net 28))
 (segment (start 68.58 78.74) (end 68.58 81.28) (width 1) (layer "B.Cu") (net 28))
 (segment (start 76.2 83.82) (end 76.2 88.9) (width 0.2) (layer "F.Cu") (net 22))
 (via (at 76.2 83.82) (size 1.6) (drill 1) (layers "F.Cu" "B.Cu") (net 22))
 (via (at 76.2 88.9) (size 1.6) (drill 1) (layers "F.Cu" "B.Cu") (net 22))
 (segment (start 68.58 88.9) (end 76.2 88.9) (width 1) (layer "B.Cu") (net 22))
 (segment (start 76.2 83.82) (end 88.9 83.82) (width 1) (layer "B.Cu") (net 22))
 (segment (start 88.9 83.82) (end 88.9 78.74) (width 1) (layer "B.Cu") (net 22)))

